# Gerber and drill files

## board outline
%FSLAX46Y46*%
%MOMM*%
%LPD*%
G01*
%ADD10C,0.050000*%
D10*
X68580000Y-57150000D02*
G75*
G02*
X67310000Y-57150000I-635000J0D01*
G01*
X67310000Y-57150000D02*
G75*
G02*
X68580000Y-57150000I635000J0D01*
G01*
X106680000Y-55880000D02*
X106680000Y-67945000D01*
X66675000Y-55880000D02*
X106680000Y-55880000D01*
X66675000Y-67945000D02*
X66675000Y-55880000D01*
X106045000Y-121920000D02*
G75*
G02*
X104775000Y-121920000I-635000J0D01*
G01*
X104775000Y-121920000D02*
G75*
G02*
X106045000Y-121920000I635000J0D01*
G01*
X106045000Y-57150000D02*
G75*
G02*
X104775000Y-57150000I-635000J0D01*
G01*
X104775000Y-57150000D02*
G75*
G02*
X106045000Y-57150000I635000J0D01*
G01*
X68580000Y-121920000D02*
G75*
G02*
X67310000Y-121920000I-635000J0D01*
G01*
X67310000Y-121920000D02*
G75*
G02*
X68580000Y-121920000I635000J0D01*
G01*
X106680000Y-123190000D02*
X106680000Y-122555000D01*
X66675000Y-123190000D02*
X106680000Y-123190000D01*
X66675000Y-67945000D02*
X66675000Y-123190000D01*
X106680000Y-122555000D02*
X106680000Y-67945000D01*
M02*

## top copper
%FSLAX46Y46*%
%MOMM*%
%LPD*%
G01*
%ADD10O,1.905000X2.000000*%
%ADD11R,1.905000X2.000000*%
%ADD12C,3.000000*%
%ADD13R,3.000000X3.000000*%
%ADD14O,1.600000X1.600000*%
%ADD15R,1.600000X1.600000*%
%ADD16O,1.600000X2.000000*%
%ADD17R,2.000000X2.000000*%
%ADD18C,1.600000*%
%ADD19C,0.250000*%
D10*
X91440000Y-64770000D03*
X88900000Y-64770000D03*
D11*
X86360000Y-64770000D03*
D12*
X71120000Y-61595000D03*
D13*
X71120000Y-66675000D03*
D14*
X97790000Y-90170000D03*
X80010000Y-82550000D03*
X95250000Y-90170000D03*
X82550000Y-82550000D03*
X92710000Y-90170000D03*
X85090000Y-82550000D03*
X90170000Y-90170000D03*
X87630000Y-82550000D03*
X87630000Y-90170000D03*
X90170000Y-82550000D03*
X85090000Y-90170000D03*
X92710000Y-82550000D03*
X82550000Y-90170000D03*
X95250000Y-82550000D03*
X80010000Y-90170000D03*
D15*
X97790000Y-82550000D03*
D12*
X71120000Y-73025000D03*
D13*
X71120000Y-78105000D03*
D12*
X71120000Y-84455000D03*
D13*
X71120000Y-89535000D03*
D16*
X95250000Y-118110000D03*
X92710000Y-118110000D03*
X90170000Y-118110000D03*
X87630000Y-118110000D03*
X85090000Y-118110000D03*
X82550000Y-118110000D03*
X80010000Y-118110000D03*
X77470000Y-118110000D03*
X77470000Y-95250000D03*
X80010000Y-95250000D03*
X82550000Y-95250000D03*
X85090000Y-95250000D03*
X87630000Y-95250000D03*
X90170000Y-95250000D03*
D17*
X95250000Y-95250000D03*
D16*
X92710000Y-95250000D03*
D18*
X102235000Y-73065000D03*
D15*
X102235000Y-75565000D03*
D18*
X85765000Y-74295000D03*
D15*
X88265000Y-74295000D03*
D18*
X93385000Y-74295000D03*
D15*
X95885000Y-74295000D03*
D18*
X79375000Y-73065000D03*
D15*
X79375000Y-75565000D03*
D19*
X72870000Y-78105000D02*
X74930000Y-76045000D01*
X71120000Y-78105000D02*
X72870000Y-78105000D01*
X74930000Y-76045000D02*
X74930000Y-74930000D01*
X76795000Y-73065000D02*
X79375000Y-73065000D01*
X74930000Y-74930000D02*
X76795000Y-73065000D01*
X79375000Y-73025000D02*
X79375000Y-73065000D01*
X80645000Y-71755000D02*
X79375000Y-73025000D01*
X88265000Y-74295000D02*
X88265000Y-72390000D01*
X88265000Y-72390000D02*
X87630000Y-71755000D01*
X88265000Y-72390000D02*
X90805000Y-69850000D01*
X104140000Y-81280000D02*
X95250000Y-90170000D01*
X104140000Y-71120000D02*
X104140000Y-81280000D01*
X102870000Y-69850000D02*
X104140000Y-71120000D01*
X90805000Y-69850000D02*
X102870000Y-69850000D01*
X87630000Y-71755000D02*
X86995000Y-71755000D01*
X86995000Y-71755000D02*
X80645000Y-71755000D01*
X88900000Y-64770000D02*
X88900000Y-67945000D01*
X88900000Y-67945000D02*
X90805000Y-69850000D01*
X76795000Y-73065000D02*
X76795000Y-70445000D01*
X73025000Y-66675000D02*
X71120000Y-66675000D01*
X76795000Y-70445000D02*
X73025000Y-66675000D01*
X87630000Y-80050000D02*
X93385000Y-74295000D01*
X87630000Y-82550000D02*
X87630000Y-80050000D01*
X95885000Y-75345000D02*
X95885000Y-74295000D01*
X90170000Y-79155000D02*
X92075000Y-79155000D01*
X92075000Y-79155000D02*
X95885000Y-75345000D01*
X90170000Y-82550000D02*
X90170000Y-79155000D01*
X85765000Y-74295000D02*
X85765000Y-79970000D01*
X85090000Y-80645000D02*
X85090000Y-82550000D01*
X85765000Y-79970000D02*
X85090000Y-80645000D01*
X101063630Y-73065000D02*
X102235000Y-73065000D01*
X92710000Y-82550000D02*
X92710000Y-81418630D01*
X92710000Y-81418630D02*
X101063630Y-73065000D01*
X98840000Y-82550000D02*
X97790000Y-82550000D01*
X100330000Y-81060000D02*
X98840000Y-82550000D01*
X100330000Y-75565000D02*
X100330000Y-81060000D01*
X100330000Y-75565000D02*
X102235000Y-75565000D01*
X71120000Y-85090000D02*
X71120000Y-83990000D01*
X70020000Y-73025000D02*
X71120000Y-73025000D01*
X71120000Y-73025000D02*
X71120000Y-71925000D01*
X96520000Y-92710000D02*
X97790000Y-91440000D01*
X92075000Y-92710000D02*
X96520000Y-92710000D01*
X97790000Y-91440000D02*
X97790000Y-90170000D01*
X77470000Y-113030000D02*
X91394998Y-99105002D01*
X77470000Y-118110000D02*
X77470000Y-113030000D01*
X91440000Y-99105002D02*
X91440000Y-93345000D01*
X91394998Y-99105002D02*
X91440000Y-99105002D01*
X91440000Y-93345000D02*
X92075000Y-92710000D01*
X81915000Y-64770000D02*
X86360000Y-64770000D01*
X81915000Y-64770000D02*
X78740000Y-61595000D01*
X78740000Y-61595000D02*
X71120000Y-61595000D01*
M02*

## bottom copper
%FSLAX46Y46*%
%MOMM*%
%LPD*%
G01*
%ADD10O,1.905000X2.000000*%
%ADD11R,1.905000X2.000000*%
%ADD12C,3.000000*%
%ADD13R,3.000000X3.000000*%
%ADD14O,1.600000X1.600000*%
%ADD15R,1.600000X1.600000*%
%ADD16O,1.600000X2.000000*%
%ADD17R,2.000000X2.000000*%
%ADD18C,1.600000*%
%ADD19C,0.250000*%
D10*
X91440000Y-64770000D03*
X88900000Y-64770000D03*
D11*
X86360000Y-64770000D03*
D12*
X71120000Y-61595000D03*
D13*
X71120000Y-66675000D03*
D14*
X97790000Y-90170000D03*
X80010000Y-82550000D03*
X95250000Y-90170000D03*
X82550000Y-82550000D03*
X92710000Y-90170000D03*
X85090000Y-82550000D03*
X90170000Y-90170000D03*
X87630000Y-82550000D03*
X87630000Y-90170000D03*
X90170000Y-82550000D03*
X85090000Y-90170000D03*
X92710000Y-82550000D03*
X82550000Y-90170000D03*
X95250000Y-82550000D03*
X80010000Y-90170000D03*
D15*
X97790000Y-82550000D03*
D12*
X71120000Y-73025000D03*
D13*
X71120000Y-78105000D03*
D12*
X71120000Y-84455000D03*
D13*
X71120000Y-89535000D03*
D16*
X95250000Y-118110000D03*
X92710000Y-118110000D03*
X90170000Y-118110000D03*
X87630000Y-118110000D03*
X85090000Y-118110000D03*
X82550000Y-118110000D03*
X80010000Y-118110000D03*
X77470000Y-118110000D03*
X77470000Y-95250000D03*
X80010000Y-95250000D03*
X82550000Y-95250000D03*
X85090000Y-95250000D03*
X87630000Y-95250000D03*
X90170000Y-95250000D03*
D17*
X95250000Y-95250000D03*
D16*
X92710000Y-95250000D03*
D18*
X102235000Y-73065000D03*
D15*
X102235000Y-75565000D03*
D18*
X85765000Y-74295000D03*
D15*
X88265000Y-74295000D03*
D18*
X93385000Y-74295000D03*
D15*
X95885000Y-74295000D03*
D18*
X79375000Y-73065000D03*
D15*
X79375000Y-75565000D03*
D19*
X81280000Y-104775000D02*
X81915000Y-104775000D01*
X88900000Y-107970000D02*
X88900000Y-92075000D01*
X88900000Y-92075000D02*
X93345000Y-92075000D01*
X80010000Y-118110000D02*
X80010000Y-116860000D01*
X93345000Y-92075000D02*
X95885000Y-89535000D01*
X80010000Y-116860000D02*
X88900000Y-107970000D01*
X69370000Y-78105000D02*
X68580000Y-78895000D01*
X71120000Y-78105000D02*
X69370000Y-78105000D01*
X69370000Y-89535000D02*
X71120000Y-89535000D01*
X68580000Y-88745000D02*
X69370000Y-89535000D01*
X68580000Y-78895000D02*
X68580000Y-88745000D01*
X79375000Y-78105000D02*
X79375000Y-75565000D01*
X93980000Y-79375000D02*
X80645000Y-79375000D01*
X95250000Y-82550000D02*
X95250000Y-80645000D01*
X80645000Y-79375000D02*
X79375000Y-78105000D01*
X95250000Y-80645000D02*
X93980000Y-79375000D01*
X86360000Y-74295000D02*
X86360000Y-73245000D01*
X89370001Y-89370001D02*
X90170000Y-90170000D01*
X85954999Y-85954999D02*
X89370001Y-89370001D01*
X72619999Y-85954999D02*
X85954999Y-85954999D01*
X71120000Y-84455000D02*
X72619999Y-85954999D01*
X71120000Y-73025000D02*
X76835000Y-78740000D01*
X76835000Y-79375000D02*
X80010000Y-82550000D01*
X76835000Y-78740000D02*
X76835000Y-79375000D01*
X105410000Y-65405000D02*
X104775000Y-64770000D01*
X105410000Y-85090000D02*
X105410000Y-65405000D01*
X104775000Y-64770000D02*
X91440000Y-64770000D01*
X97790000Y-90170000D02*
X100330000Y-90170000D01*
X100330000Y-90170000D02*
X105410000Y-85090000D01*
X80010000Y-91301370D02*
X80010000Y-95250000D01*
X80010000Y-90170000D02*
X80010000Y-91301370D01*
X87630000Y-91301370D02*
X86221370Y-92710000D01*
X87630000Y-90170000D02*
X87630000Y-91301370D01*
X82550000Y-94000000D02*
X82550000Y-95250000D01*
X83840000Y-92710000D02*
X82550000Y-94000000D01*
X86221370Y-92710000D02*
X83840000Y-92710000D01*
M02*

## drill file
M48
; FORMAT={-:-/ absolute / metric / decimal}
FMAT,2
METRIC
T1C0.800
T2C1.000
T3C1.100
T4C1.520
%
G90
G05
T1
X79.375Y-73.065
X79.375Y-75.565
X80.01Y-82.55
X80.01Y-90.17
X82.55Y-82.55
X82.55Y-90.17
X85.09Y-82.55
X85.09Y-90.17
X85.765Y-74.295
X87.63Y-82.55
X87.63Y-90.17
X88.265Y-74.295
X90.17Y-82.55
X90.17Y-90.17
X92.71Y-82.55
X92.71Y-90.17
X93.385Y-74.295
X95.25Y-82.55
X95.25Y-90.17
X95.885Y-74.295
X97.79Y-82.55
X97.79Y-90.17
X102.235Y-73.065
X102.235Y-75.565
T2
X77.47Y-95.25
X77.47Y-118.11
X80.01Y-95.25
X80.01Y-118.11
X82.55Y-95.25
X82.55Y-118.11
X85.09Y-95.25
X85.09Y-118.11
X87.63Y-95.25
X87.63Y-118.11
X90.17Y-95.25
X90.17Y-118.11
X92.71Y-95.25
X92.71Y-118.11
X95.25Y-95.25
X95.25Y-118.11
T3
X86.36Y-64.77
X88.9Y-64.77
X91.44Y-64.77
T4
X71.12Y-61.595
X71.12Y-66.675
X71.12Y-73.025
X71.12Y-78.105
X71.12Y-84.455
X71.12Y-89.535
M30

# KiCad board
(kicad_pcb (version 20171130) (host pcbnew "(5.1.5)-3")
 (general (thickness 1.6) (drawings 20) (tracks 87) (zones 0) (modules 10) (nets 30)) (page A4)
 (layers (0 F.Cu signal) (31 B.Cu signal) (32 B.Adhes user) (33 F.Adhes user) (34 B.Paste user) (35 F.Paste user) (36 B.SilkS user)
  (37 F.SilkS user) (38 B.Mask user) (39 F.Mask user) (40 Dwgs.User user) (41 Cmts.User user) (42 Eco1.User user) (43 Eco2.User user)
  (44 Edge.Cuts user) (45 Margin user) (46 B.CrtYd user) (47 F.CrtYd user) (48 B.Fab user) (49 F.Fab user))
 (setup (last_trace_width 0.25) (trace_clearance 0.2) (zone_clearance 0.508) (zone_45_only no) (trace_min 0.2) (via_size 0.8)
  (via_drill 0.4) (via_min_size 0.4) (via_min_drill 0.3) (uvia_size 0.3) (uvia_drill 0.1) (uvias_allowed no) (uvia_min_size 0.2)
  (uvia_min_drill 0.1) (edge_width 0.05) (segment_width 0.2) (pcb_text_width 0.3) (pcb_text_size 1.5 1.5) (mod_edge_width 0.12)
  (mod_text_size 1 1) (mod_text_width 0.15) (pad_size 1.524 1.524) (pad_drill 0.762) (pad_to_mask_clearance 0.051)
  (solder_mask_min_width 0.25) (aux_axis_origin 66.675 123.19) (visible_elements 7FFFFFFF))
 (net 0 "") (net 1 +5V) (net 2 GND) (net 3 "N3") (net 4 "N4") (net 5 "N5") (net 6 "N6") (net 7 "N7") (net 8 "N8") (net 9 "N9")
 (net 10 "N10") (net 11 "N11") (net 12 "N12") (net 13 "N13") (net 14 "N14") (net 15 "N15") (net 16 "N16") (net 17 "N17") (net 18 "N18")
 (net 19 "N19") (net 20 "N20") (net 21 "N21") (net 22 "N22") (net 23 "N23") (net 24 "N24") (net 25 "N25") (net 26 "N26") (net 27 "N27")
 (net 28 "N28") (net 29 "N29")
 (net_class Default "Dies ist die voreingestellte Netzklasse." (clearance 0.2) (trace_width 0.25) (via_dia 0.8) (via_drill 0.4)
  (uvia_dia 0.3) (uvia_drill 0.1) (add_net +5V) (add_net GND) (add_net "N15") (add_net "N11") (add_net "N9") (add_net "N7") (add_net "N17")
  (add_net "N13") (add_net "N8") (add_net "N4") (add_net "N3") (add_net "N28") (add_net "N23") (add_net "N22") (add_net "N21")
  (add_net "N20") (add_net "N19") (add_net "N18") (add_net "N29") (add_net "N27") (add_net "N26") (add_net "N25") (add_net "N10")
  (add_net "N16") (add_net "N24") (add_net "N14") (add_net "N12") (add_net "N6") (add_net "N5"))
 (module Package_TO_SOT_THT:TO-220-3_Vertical (layer F.Cu) (at 86.36 64.77)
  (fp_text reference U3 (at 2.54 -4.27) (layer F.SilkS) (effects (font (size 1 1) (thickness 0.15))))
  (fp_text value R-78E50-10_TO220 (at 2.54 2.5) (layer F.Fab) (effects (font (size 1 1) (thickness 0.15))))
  (pad 3 thru_hole oval (at 5.08 0) (size 1.905 2) (drill 1.1) (layers *.Cu *.Mask) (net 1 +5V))
  (pad 2 thru_hole oval (at 2.54 0) (size 1.905 2) (drill 1.1) (layers *.Cu *.Mask) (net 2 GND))
  (pad 1 thru_hole rect (at 0 0) (size 1.905 2) (drill 1.1) (layers *.Cu *.Mask) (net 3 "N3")))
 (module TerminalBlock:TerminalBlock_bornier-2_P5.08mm (layer F.Cu) (at 71.12 66.675 90)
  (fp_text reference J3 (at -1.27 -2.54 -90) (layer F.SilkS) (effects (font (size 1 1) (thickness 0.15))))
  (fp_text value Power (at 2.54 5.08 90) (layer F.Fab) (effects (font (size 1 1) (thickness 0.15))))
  (pad 2 thru_hole circle (at 5.08 0 90) (size 3 3) (drill 1.52) (layers *.Cu *.Mask) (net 3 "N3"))
  (pad 1 thru_hole rect (at 0 0 90) (size 3 3) (drill 1.52) (layers *.Cu *.Mask) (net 2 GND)))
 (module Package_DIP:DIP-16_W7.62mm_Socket (layer F.Cu) (at 97.79 82.55 270)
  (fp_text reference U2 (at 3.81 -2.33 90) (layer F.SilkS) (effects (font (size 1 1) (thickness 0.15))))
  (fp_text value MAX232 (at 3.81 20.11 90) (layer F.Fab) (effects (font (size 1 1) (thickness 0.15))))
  (pad 16 thru_hole oval (at 7.62 0 270) (size 1.6 1.6) (drill 0.8) (layers *.Cu *.Mask) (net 1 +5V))
  (pad 8 thru_hole oval (at 0 17.78 270) (size 1.6 1.6) (drill 0.8) (layers *.Cu *.Mask) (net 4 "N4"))
  (pad 15 thru_hole oval (at 7.62 2.54 270) (size 1.6 1.6) (drill 0.8) (layers *.Cu *.Mask) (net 2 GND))
  (pad 7 thru_hole oval (at 0 15.24 270) (size 1.6 1.6) (drill 0.8) (layers *.Cu *.Mask) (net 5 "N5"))
  (pad 14 thru_hole oval (at 7.62 5.08 270) (size 1.6 1.6) (drill 0.8) (layers *.Cu *.Mask) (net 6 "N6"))
  (pad 6 thru_hole oval (at 0 12.7 270) (size 1.6 1.6) (drill 0.8) (layers *.Cu *.Mask) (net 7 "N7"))
  (pad 13 thru_hole oval (at 7.62 7.62 270) (size 1.6 1.6) (drill 0.8) (layers *.Cu *.Mask) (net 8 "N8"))
  (pad 5 thru_hole oval (at 0 10.16 270) (size 1.6 1.6) (drill 0.8) (layers *.Cu *.Mask) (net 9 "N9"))
  (pad 12 thru_hole oval (at 7.62 10.16 270) (size 1.6 1.6) (drill 0.8) (layers *.Cu *.Mask) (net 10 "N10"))
  (pad 4 thru_hole oval (at 0 7.62 270) (size 1.6 1.6) (drill 0.8) (layers *.Cu *.Mask) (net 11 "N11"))
  (pad 11 thru_hole oval (at 7.62 12.7 270) (size 1.6 1.6) (drill 0.8) (layers *.Cu *.Mask) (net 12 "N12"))
  (pad 3 thru_hole oval (at 0 5.08 270) (size 1.6 1.6) (drill 0.8) (layers *.Cu *.Mask) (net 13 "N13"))
  (pad 10 thru_hole oval (at 7.62 15.24 270) (size 1.6 1.6) (drill 0.8) (layers *.Cu *.Mask) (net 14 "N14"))
  (pad 2 thru_hole oval (at 0 2.54 270) (size 1.6 1.6) (drill 0.8) (layers *.Cu *.Mask) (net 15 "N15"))
  (pad 9 thru_hole oval (at 7.62 17.78 270) (size 1.6 1.6) (drill 0.8) (layers *.Cu *.Mask) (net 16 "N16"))
  (pad 1 thru_hole rect (at 0 0 270) (size 1.6 1.6) (drill 0.8) (layers *.Cu *.Mask) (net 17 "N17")))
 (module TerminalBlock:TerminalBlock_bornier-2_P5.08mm (layer F.Cu) (at 71.12 78.105 90)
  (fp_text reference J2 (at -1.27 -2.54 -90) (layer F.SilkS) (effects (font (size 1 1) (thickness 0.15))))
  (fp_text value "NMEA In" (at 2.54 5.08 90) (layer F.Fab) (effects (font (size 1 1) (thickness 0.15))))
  (pad 2 thru_hole circle (at 5.08 0 90) (size 3 3) (drill 1.52) (layers *.Cu *.Mask) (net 4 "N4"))
  (pad 1 thru_hole rect (at 0 0 90) (size 3 3) (drill 1.52) (layers *.Cu *.Mask) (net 2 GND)))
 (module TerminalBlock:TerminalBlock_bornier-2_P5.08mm (layer F.Cu) (at 71.12 89.535 90)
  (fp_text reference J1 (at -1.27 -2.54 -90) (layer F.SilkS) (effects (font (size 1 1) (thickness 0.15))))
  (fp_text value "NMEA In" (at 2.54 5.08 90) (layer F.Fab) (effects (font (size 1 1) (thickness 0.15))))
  (pad 2 thru_hole circle (at 5.08 0 90) (size 3 3) (drill 1.52) (layers *.Cu *.Mask) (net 8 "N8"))
  (pad 1 thru_hole rect (at 0 0 90) (size 3 3) (drill 1.52) (layers *.Cu *.Mask) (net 2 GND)))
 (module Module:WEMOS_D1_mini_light (layer F.Cu) (at 95.25 95.25 270)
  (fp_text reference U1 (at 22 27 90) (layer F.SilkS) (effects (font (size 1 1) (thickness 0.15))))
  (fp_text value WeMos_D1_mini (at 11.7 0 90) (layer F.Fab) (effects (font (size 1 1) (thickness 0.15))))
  (pad 16 thru_hole oval (at 22.86 0 270) (size 2 1.6) (drill 1) (layers *.Cu *.Mask) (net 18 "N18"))
  (pad 15 thru_hole oval (at 22.86 2.54 270) (size 2 1.6) (drill 1) (layers *.Cu *.Mask) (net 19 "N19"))
  (pad 14 thru_hole oval (at 22.86 5.08 270) (size 2 1.6) (drill 1) (layers *.Cu *.Mask) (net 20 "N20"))
  (pad 13 thru_hole oval (at 22.86 7.62 270) (size 2 1.6) (drill 1) (layers *.Cu *.Mask) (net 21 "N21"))
  (pad 12 thru_hole oval (at 22.86 10.16 270) (size 2 1.6) (drill 1) (layers *.Cu *.Mask) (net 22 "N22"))
  (pad 11 thru_hole oval (at 22.86 12.7 270) (size 2 1.6) (drill 1) (layers *.Cu *.Mask) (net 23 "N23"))
  (pad 10 thru_hole oval (at 22.86 15.24 270) (size 2 1.6) (drill 1) (layers *.Cu *.Mask) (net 2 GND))
  (pad 9 thru_hole oval (at 22.86 17.78 270) (size 2 1.6) (drill 1) (layers *.Cu *.Mask) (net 1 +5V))
  (pad 8 thru_hole oval (at 0 17.78 270) (size 2 1.6) (drill 1) (layers *.Cu *.Mask) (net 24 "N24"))
  (pad 7 thru_hole oval (at 0 15.24 270) (size 2 1.6) (drill 1) (layers *.Cu *.Mask) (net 16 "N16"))
  (pad 6 thru_hole oval (at 0 12.7 270) (size 2 1.6) (drill 1) (layers *.Cu *.Mask) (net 10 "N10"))
  (pad 5 thru_hole oval (at 0 10.16 270) (size 2 1.6) (drill 1) (layers *.Cu *.Mask) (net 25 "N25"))
  (pad 4 thru_hole oval (at 0 7.62 270) (size 2 1.6) (drill 1) (layers *.Cu *.Mask) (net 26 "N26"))
  (pad 3 thru_hole oval (at 0 5.08 270) (size 2 1.6) (drill 1) (layers *.Cu *.Mask) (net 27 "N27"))
  (pad 1 thru_hole rect (at 0 0 270) (size 2 2) (drill 1) (layers *.Cu *.Mask) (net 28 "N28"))
  (pad 2 thru_hole oval (at 0 2.54 270) (size 2 1.6) (drill 1) (layers *.Cu *.Mask) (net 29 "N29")))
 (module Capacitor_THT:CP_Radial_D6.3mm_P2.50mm (layer F.Cu) (at 102.235 75.565 90)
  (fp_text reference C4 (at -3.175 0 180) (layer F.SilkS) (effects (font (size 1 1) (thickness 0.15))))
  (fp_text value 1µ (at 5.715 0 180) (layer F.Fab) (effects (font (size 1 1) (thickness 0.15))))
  (pad 2 thru_hole circle (at 2.5 0 90) (size 1.6 1.6) (drill 0.8) (layers *.Cu *.Mask) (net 13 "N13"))
  (pad 1 thru_hole rect (at 0 0 90) (size 1.6 1.6) (drill 0.8) (layers *.Cu *.Mask) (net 17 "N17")))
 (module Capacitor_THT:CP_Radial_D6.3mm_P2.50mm (layer F.Cu) (at 88.265 74.295 180)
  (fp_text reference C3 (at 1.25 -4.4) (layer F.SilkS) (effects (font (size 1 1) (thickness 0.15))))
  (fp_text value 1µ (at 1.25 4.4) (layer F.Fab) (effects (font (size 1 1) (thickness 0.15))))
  (pad 2 thru_hole circle (at 2.5 0 180) (size 1.6 1.6) (drill 0.8) (layers *.Cu *.Mask) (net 7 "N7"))
  (pad 1 thru_hole rect (at 0 0 180) (size 1.6 1.6) (drill 0.8) (layers *.Cu *.Mask) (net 2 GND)))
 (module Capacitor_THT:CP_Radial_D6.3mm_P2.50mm (layer F.Cu) (at 95.885 74.295 180)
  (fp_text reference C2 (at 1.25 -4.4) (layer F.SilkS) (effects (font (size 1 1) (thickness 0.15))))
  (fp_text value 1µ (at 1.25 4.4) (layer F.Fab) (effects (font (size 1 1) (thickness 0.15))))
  (pad 2 thru_hole circle (at 2.5 0 180) (size 1.6 1.6) (drill 0.8) (layers *.Cu *.Mask) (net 9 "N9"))
  (pad 1 thru_hole rect (at 0 0 180) (size 1.6 1.6) (drill 0.8) (layers *.Cu *.Mask) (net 11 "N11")))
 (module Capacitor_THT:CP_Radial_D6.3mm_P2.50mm (layer F.Cu) (at 79.375 75.565 90)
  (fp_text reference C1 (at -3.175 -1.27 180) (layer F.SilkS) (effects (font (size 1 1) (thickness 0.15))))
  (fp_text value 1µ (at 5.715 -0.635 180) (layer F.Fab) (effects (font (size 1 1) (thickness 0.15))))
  (pad 2 thru_hole circle (at 2.5 0 90) (size 1.6 1.6) (drill 0.8) (layers *.Cu *.Mask) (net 2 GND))
  (pad 1 thru_hole rect (at 0 0 90) (size 1.6 1.6) (drill 0.8) (layers *.Cu *.Mask) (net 15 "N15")))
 (gr_circle (center 67.945 57.15) (end 68.58 57.15) (layer Edge.Cuts) (width 0.05))
 (gr_line (start 106.68 55.88) (end 106.68 67.945) (layer Edge.Cuts) (width 0.05))
 (gr_line (start 66.675 55.88) (end 106.68 55.88) (layer Edge.Cuts) (width 0.05))
 (gr_line (start 66.675 67.945) (end 66.675 55.88) (layer Edge.Cuts) (width 0.05))
 (gr_circle (center 105.41 121.92) (end 106.045 121.92) (layer Edge.Cuts) (width 0.05))
 (gr_circle (center 105.41 57.15) (end 106.045 57.15) (layer Edge.Cuts) (width 0.05))
 (gr_circle (center 67.945 121.92) (end 67.945 121.285) (layer Edge.Cuts) (width 0.05))
 (gr_line (start 106.68 123.19) (end 106.68 122.555) (layer Edge.Cuts) (width 0.05))
 (gr_line (start 66.675 123.19) (end 106.68 123.19) (layer Edge.Cuts) (width 0.05))
 (gr_line (start 66.675 67.945) (end 66.675 123.19) (layer Edge.Cuts) (width 0.05))
 (gr_line (start 106.68 122.555) (end 106.68 67.945) (layer Edge.Cuts) (width 0.05))
 (segment (start 81.28 104.775) (end 81.915 104.775) (width 0.25) (layer B.Cu) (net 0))
 (segment (start 88.9 107.97) (end 88.9 92.075) (width 0.25) (layer B.Cu) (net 2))
 (segment (start 88.9 92.075) (end 93.345 92.075) (width 0.25) (layer B.Cu) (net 2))
 (segment (start 80.01 118.11) (end 80.01 116.86) (width 0.25) (layer B.Cu) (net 2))
 (segment (start 93.345 92.075) (end 95.885 89.535) (width 0.25) (layer B.Cu) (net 2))
 (segment (start 80.01 116.86) (end 88.9 107.97) (width 0.25) (layer B.Cu) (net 2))
 (segment (start 72.87 78.105) (end 74.93 76.045) (width 0.25) (layer F.Cu) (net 2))
 (segment (start 71.12 78.105) (end 72.87 78.105) (width 0.25) (layer F.Cu) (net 2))
 (segment (start 74.93 76.045) (end 74.93 74.93) (width 0.25) (layer F.Cu) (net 2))
 (segment (start 76.795 73.065) (end 79.375 73.065) (width 0.25) (layer F.Cu) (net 2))
 (segment (start 74.93 74.93) (end 76.795 73.065) (width 0.25) (layer F.Cu) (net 2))
 (segment (start 79.375 73.025) (end 79.375 73.065) (width 0.25) (layer F.Cu) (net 2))
 (segment (start 80.645 71.755) (end 79.375 73.025) (width 0.25) (layer F.Cu) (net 2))
 (segment (start 88.265 74.295) (end 88.265 72.39) (width 0.25) (layer F.Cu) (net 2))
 (segment (start 88.265 72.39) (end 87.63 71.755) (width 0.25) (layer F.Cu) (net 2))
 (segment (start 88.265 72.39) (end 90.805 69.85) (width 0.25) (layer F.Cu) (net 2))
 (segment (start 104.14 81.28) (end 95.25 90.17) (width 0.25) (layer F.Cu) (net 2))
 (segment (start 104.14 71.12) (end 104.14 81.28) (width 0.25) (layer F.Cu) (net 2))
 (segment (start 102.87 69.85) (end 104.14 71.12) (width 0.25) (layer F.Cu) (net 2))
 (segment (start 90.805 69.85) (end 102.87 69.85) (width 0.25) (layer F.Cu) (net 2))
 (segment (start 69.37 78.105) (end 68.58 78.895) (width 0.25) (layer B.Cu) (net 2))
 (segment (start 71.12 78.105) (end 69.37 78.105) (width 0.25) (layer B.Cu) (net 2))
 (segment (start 69.37 89.535) (end 71.12 89.535) (width 0.25) (layer B.Cu) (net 2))
 (segment (start 68.58 88.745) (end 69.37 89.535) (width 0.25) (layer B.Cu) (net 2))
 (segment (start 68.58 78.895) (end 68.58 88.745) (width 0.25) (layer B.Cu) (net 2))
 (segment (start 87.63 71.755) (end 86.995 71.755) (width 0.25) (layer F.Cu) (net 2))
 (segment (start 86.995 71.755) (end 80.645 71.755) (width 0.25) (layer F.Cu) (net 2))
 (segment (start 88.9 64.77) (end 88.9 67.945) (width 0.25) (layer F.Cu) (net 2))
 (segment (start 88.9 67.945) (end 90.805 69.85) (width 0.25) (layer F.Cu) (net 2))
 (segment (start 76.795 73.065) (end 76.795 70.445) (width 0.25) (layer F.Cu) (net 2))
 (segment (start 73.025 66.675) (end 71.12 66.675) (width 0.25) (layer F.Cu) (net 2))
 (segment (start 76.795 70.445) (end 73.025 66.675) (width 0.25) (layer F.Cu) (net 2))
 (segment (start 79.375 78.105) (end 79.375 75.565) (width 0.25) (layer B.Cu) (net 15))
 (segment (start 93.98 79.375) (end 80.645 79.375) (width 0.25) (layer B.Cu) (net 15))
 (segment (start 95.25 82.55) (end 95.25 80.645) (width 0.25) (layer B.Cu) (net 15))
 (segment (start 80.645 79.375) (end 79.375 78.105) (width 0.25) (layer B.Cu) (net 15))
 (segment (start 95.25 80.645) (end 93.98 79.375) (width 0.25) (layer B.Cu) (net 15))
 (segment (start 87.63 80.05) (end 93.385 74.295) (width 0.25) (layer F.Cu) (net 9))
 (segment (start 87.63 82.55) (end 87.63 80.05) (width 0.25) (layer F.Cu) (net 9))
 (segment (start 95.885 75.345) (end 95.885 74.295) (width 0.25) (layer F.Cu) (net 11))
 (segment (start 90.17 79.155) (end 92.075 79.155) (width 0.25) (layer F.Cu) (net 11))
 (segment (start 92.075 79.155) (end 95.885 75.345) (width 0.25) (layer F.Cu) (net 11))
 (segment (start 90.17 82.55) (end 90.17 79.155) (width 0.25) (layer F.Cu) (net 11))
 (segment (start 86.36 74.295) (end 86.36 73.245) (width 0.25) (layer B.Cu) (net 7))
 (segment (start 85.765 74.295) (end 85.765 79.97) (width 0.25) (layer F.Cu) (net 7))
 (segment (start 85.09 80.645) (end 85.09 82.55) (width 0.25) (layer F.Cu) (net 7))
 (segment (start 85.765 79.97) (end 85.09 80.645) (width 0.25) (layer F.Cu) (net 7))
 (segment (start 101.06363 73.065) (end 102.235 73.065) (width 0.25) (layer F.Cu) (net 13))
 (segment (start 92.71 82.55) (end 92.71 81.41863) (width 0.25) (layer F.Cu) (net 13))
 (segment (start 92.71 81.41863) (end 101.06363 73.065) (width 0.25) (layer F.Cu) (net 13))
 (segment (start 98.84 82.55) (end 97.79 82.55) (width 0.25) (layer F.Cu) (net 17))
 (segment (start 100.33 81.06) (end 98.84 82.55) (width 0.25) (layer F.Cu) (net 17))
 (segment (start 100.33 75.565) (end 100.33 81.06) (width 0.25) (layer F.Cu) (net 17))
 (segment (start 100.33 75.565) (end 102.235 75.565) (width 0.25) (layer F.Cu) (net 17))
 (segment (start 71.12 85.09) (end 71.12 83.99) (width 0.25) (layer F.Cu) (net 8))
 (segment (start 89.370001 89.370001) (end 90.17 90.17) (width 0.25) (layer B.Cu) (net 8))
 (segment (start 85.954999 85.954999) (end 89.370001 89.370001) (width 0.25) (layer B.Cu) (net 8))
 (segment (start 72.619999 85.954999) (end 85.954999 85.954999) (width 0.25) (layer B.Cu) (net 8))
 (segment (start 71.12 84.455) (end 72.619999 85.954999) (width 0.25) (layer B.Cu) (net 8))
 (segment (start 70.02 73.025) (end 71.12 73.025) (width 0.25) (layer F.Cu) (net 4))
 (segment (start 71.12 73.025) (end 71.12 71.925) (width 0.25) (layer F.Cu) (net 4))
 (segment (start 71.12 73.025) (end 76.835 78.74) (width 0.25) (layer B.Cu) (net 4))
 (segment (start 76.835 79.375) (end 80.01 82.55) (width 0.25) (layer B.Cu) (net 4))
 (segment (start 76.835 78.74) (end 76.835 79.375) (width 0.25) (layer B.Cu) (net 4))
 (segment (start 96.52 92.71) (end 97.79 91.44) (width 0.25) (layer F.Cu) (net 1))
 (segment (start 92.075 92.71) (end 96.52 92.71) (width 0.25) (layer F.Cu) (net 1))
 (segment (start 97.79 91.44) (end 97.79 90.17) (width 0.25) (layer F.Cu) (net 1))
 (segment (start 77.47 113.03) (end 91.394998 99.105002) (width 0.25) (layer F.Cu) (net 1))
 (segment (start 77.47 118.11) (end 77.47 113.03) (width 0.25) (layer F.Cu) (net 1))
 (segment (start 91.44 99.105002) (end 91.44 93.345) (width 0.25) (layer F.Cu) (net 1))
 (segment (start 91.394998 99.105002) (end 91.44 99.105002) (width 0.25) (layer F.Cu) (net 1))
 (segment (start 91.44 93.345) (end 92.075 92.71) (width 0.25) (layer F.Cu) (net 1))
 (segment (start 105.41 65.405) (end 104.775 64.77) (width 0.25) (layer B.Cu) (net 1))
 (segment (start 105.41 85.09) (end 105.41 65.405) (width 0.25) (layer B.Cu) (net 1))
 (segment (start 104.775 64.77) (end 91.44 64.77) (width 0.25) (layer B.Cu) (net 1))
 (segment (start 97.79 90.17) (end 100.33 90.17) (width 0.25) (layer B.Cu) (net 1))
 (segment (start 100.33 90.17) (end 105.41 85.09) (width 0.25) (layer B.Cu) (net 1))
 (segment (start 80.01 91.30137) (end 80.01 95.25) (width 0.25) (layer B.Cu) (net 16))
 (segment (start 80.01 90.17) (end 80.01 91.30137) (width 0.25) (layer B.Cu) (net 16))
 (segment (start 87.63 91.30137) (end 86.22137 92.71) (width 0.25) (layer B.Cu) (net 10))
 (segment (start 87.63 90.17) (end 87.63 91.30137) (width 0.25) (layer B.Cu) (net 10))
 (segment (start 82.55 94) (end 82.55 95.25) (width 0.25) (layer B.Cu) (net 10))
 (segment (start 83.84 92.71) (end 82.55 94) (width 0.25) (layer B.Cu) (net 10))
 (segment (start 86.22137 92.71) (end 83.84 92.71) (width 0.25) (layer B.Cu) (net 10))
 (segment (start 81.915 64.77) (end 86.36 64.77) (width 0.25) (layer F.Cu) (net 3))
 (segment (start 81.915 64.77) (end 78.74 61.595) (width 0.25) (layer F.Cu) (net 3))
 (segment (start 78.74 61.595) (end 71.12 61.595) (width 0.25) (layer F.Cu) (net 3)))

